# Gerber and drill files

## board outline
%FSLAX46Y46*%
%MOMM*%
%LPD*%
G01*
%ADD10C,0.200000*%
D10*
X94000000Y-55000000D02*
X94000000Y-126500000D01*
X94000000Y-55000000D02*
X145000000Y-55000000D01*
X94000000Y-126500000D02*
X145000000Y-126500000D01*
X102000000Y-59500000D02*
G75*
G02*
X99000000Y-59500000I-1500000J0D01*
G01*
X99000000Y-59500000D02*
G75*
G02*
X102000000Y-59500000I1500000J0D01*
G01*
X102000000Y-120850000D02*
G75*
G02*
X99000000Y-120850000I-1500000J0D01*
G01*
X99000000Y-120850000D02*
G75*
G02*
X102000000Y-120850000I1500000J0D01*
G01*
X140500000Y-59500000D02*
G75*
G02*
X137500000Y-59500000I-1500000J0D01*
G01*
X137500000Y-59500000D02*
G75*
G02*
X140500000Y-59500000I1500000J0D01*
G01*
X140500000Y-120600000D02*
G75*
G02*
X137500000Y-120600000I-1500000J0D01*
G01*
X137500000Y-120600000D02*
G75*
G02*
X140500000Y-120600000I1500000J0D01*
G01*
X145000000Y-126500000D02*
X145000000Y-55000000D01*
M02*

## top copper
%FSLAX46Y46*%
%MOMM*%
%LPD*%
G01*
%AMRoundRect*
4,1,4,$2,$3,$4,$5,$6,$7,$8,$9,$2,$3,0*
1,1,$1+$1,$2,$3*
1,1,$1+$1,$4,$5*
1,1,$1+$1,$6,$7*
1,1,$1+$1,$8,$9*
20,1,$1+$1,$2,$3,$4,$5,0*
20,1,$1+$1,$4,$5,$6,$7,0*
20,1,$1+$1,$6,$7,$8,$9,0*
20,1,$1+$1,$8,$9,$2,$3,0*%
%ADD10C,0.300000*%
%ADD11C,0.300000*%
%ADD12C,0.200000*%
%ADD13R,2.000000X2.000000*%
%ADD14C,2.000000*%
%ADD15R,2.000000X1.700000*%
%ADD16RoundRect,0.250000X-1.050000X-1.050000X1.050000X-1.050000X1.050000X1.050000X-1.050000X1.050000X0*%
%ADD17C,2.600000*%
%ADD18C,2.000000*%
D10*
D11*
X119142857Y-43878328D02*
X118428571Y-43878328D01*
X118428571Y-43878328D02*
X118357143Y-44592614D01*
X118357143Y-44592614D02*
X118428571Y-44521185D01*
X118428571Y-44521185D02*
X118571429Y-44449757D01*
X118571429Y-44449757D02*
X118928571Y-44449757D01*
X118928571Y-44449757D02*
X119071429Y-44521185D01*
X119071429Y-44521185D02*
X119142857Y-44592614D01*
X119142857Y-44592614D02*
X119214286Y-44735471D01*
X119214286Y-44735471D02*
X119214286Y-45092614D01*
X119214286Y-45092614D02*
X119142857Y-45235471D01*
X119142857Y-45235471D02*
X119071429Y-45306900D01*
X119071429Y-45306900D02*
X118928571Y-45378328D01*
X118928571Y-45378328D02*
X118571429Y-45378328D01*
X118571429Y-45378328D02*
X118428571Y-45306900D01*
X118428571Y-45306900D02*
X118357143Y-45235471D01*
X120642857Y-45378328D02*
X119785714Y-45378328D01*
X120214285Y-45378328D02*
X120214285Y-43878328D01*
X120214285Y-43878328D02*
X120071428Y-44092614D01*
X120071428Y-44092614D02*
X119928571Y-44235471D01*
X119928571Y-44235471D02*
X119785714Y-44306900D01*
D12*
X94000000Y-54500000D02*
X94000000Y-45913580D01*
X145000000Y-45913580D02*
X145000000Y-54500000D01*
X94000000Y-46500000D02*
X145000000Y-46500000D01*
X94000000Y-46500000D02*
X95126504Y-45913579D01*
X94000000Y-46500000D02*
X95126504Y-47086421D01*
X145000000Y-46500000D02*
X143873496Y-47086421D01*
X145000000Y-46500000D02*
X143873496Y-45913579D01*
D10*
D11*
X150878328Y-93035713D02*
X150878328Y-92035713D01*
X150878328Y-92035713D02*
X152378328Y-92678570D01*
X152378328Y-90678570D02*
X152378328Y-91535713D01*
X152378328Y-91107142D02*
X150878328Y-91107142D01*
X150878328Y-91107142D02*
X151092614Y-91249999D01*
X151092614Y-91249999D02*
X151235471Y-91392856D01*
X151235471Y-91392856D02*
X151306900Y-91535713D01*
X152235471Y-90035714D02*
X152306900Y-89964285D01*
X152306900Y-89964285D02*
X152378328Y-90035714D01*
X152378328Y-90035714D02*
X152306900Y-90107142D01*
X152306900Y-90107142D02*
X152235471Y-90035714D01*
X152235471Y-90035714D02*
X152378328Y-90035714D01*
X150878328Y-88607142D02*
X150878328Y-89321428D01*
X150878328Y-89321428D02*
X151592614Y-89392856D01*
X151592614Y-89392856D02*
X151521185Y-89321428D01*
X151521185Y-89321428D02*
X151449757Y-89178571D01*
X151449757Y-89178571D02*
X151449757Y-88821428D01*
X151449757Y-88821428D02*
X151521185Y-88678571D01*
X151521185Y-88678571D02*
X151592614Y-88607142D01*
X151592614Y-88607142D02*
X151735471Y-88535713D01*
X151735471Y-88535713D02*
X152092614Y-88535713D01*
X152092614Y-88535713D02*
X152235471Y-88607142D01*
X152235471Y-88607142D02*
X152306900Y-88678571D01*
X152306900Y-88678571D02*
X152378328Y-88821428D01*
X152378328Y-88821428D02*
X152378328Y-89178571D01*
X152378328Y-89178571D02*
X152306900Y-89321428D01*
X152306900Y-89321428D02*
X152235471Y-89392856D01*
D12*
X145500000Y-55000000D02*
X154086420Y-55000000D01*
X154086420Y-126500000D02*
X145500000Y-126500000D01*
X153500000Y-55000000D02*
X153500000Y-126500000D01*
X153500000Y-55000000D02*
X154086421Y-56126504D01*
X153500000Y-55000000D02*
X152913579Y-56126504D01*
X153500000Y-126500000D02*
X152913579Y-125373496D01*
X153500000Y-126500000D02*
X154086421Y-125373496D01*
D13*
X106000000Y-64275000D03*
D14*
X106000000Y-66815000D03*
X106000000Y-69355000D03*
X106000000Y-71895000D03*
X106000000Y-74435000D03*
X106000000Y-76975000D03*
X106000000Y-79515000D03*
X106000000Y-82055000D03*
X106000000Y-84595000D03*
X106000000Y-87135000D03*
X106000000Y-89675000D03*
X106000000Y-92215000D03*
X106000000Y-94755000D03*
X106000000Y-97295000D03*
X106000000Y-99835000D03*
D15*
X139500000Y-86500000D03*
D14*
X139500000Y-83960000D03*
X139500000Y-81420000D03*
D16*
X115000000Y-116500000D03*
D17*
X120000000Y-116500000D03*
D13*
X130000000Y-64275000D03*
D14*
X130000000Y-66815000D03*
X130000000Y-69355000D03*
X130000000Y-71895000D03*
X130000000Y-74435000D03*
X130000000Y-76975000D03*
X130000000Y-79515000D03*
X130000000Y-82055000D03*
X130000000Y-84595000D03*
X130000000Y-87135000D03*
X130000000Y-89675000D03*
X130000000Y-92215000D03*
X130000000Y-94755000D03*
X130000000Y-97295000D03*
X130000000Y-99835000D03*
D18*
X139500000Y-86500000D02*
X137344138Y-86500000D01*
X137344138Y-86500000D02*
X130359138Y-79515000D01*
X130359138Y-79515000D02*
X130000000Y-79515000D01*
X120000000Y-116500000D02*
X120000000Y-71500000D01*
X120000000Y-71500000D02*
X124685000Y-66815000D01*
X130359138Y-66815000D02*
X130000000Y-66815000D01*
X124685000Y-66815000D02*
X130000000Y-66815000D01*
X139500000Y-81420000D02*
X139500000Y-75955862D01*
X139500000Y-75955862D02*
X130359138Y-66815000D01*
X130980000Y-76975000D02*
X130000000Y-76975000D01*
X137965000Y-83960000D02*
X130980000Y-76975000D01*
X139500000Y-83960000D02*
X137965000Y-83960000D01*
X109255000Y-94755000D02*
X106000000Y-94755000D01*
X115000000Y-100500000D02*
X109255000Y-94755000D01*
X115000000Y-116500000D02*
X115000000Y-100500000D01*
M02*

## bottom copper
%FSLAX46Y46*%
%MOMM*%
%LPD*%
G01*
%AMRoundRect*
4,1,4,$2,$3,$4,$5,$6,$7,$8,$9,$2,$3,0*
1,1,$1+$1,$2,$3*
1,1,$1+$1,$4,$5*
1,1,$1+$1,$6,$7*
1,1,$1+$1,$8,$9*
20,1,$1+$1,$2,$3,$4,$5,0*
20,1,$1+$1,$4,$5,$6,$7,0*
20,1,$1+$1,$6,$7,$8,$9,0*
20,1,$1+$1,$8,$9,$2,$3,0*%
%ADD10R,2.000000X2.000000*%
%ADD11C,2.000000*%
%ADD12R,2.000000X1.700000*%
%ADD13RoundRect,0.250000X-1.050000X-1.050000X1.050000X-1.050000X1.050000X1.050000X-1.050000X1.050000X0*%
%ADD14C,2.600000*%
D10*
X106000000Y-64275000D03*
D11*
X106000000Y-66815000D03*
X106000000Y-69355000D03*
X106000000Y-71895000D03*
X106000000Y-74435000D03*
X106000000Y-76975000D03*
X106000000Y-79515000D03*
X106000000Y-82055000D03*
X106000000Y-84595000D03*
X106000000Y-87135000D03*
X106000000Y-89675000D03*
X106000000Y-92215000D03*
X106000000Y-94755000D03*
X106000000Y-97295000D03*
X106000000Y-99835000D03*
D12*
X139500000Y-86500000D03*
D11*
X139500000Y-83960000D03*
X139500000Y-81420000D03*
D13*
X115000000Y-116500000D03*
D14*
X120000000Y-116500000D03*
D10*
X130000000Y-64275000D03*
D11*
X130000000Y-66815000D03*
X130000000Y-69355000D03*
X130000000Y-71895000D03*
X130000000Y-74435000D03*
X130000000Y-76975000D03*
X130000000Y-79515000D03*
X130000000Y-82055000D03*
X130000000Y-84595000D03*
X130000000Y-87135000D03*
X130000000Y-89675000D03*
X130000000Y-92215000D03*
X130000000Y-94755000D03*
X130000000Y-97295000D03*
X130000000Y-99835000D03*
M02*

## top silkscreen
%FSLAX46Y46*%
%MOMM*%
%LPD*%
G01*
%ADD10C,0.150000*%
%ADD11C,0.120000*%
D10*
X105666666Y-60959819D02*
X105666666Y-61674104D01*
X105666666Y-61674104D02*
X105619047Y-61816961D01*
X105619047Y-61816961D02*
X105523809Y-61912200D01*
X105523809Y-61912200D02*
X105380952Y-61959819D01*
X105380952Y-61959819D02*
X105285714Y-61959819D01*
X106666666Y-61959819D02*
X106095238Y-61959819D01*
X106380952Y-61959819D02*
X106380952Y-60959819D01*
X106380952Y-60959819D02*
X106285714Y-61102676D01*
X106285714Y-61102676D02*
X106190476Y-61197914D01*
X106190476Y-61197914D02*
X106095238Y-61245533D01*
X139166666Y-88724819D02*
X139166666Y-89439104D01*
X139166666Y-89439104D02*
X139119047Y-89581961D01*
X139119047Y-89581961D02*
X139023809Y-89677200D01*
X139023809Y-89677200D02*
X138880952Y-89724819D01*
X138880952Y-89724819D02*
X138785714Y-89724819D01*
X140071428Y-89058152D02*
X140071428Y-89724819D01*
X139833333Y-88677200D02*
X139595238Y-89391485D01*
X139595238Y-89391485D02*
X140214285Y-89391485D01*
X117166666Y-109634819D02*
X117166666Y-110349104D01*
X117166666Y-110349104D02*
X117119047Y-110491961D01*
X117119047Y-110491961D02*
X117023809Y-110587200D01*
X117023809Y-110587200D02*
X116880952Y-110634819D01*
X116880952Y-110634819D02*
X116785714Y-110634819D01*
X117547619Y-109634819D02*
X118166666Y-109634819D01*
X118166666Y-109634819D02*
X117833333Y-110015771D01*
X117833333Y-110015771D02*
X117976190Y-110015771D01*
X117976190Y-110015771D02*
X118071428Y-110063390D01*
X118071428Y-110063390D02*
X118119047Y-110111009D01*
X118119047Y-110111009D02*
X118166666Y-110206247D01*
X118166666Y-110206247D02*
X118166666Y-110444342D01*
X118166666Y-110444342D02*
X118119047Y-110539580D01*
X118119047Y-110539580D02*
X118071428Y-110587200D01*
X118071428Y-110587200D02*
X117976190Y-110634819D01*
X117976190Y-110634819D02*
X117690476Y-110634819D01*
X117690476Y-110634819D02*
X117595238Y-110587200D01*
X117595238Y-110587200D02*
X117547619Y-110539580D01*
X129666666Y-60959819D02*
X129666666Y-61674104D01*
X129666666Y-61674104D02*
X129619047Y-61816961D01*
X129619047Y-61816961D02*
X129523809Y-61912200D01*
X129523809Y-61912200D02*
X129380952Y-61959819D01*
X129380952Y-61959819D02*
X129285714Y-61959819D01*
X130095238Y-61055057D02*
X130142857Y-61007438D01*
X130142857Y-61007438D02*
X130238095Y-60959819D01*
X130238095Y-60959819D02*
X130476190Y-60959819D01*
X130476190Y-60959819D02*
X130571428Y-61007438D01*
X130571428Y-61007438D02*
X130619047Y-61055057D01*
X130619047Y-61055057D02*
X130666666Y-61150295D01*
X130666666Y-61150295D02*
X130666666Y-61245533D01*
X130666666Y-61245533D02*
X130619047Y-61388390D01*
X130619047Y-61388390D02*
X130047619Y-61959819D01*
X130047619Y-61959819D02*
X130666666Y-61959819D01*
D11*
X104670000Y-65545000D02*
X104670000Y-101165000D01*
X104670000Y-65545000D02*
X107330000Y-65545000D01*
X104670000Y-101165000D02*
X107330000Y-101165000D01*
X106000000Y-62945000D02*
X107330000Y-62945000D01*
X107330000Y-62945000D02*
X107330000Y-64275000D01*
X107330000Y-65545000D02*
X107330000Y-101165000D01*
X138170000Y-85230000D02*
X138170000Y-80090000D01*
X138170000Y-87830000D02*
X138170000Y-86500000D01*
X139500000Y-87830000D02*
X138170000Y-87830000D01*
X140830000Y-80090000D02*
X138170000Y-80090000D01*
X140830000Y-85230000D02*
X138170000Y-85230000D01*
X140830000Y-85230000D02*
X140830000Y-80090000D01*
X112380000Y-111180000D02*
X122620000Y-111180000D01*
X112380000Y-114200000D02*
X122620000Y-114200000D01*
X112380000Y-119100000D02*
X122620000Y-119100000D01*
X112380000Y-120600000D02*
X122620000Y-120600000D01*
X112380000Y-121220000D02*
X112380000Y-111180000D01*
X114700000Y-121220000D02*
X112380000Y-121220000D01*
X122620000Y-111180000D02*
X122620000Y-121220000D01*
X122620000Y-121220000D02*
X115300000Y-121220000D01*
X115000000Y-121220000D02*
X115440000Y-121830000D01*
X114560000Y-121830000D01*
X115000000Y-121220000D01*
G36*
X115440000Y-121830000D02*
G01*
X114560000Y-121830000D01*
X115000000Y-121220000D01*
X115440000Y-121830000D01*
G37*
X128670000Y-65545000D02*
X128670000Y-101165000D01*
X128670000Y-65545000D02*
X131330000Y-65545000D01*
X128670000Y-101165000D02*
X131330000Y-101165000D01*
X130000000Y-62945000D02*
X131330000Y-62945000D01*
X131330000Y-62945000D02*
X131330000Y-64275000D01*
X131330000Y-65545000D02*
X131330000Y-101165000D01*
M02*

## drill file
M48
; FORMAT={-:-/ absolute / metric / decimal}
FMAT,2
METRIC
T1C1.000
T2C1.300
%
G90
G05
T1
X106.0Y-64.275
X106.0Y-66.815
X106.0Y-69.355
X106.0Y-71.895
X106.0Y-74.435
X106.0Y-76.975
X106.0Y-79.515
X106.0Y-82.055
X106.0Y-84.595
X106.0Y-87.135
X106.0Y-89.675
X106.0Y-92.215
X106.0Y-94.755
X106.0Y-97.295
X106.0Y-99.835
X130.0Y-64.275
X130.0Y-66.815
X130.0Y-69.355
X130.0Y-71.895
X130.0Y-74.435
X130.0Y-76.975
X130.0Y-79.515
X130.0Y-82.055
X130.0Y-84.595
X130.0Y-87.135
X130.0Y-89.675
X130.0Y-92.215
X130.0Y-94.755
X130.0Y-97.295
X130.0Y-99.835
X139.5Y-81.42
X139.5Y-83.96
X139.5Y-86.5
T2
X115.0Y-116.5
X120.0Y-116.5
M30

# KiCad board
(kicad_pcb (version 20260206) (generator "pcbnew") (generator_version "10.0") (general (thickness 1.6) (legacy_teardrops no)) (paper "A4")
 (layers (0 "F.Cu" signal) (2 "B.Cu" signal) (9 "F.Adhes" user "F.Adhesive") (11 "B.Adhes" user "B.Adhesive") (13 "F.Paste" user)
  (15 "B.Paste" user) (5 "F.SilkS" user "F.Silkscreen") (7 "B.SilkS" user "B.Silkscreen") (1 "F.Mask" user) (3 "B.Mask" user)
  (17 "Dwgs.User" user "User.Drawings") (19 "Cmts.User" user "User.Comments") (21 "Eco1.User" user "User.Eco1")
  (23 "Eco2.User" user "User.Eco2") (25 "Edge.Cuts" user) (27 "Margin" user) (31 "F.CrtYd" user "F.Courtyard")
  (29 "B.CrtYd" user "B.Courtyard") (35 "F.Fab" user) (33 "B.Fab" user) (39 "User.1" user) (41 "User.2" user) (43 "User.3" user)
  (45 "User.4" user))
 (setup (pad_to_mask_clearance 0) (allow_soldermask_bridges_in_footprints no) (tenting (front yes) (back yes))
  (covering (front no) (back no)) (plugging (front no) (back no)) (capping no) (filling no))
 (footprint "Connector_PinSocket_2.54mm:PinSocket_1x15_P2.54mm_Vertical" (layer "F.Cu") (at 106 64.275)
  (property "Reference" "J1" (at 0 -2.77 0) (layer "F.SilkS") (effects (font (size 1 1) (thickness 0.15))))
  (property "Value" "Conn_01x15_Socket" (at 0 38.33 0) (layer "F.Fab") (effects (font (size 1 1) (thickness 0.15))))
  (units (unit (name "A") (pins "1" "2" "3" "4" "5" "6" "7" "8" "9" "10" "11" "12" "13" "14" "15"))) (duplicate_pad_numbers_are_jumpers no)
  (fp_line (start -1.33 1.27) (end -1.33 36.89) (stroke (width 0.12) (type solid)) (layer "F.SilkS"))
  (fp_line (start -1.33 1.27) (end 1.33 1.27) (stroke (width 0.12) (type solid)) (layer "F.SilkS"))
  (fp_line (start -1.33 36.89) (end 1.33 36.89) (stroke (width 0.12) (type solid)) (layer "F.SilkS"))
  (fp_line (start 0 -1.33) (end 1.33 -1.33) (stroke (width 0.12) (type solid)) (layer "F.SilkS"))
  (fp_line (start 1.33 -1.33) (end 1.33 0) (stroke (width 0.12) (type solid)) (layer "F.SilkS"))
  (fp_line (start 1.33 1.27) (end 1.33 36.89) (stroke (width 0.12) (type solid)) (layer "F.SilkS"))
  (pad "1" thru_hole rect (at 0 0) (size 2 2) (drill 1) (layers "*.Cu" "*.Mask") (remove_unused_layers no)
   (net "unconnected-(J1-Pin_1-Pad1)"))
  (pad "2" thru_hole circle (at 0 2.54) (size 2 2) (drill 1) (layers "*.Cu" "*.Mask") (remove_unused_layers no)
   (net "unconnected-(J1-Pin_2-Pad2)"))
  (pad "3" thru_hole circle (at 0 5.08) (size 2 2) (drill 1) (layers "*.Cu" "*.Mask") (remove_unused_layers no)
   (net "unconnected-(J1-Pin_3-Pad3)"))
  (pad "4" thru_hole circle (at 0 7.62) (size 2 2) (drill 1) (layers "*.Cu" "*.Mask") (remove_unused_layers no)
   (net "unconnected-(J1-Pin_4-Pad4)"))
  (pad "5" thru_hole circle (at 0 10.16) (size 2 2) (drill 1) (layers "*.Cu" "*.Mask") (remove_unused_layers no)
   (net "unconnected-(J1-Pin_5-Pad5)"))
  (pad "6" thru_hole circle (at 0 12.7) (size 2 2) (drill 1) (layers "*.Cu" "*.Mask") (remove_unused_layers no)
   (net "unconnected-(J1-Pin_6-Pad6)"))
  (pad "7" thru_hole circle (at 0 15.24) (size 2 2) (drill 1) (layers "*.Cu" "*.Mask") (remove_unused_layers no)
   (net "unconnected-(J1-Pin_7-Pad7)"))
  (pad "8" thru_hole circle (at 0 17.78) (size 2 2) (drill 1) (layers "*.Cu" "*.Mask") (remove_unused_layers no)
   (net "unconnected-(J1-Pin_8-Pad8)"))
  (pad "9" thru_hole circle (at 0 20.32) (size 2 2) (drill 1) (layers "*.Cu" "*.Mask") (remove_unused_layers no)
   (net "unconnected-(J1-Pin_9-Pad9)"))
  (pad "10" thru_hole circle (at 0 22.86) (size 2 2) (drill 1) (layers "*.Cu" "*.Mask") (remove_unused_layers no)
   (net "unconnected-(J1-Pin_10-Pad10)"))
  (pad "11" thru_hole circle (at 0 25.4) (size 2 2) (drill 1) (layers "*.Cu" "*.Mask") (remove_unused_layers no)
   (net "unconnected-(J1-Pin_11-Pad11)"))
  (pad "12" thru_hole circle (at 0 27.94) (size 2 2) (drill 1) (layers "*.Cu" "*.Mask") (remove_unused_layers no)
   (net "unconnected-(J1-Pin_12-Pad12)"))
  (pad "13" thru_hole circle (at 0 30.48) (size 2 2) (drill 1) (layers "*.Cu" "*.Mask") (remove_unused_layers no) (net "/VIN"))
  (pad "14" thru_hole circle (at 0 33.02) (size 2 2) (drill 1) (layers "*.Cu" "*.Mask") (remove_unused_layers no)
   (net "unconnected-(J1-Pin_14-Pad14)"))
  (pad "15" thru_hole circle (at 0 35.56) (size 2 2) (drill 1) (layers "*.Cu" "*.Mask") (remove_unused_layers no)
   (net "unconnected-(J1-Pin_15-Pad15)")))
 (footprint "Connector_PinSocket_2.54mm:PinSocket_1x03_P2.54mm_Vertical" (layer "F.Cu") (at 139.5 86.5 180)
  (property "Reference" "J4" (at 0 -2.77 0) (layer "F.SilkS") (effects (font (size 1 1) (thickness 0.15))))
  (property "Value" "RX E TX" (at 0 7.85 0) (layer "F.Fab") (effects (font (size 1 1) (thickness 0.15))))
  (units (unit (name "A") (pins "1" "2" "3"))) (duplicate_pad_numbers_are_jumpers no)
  (fp_line (start 1.33 1.27) (end 1.33 6.41) (stroke (width 0.12) (type solid)) (layer "F.SilkS"))
  (fp_line (start 1.33 -1.33) (end 1.33 0) (stroke (width 0.12) (type solid)) (layer "F.SilkS"))
  (fp_line (start 0 -1.33) (end 1.33 -1.33) (stroke (width 0.12) (type solid)) (layer "F.SilkS"))
  (fp_line (start -1.33 6.41) (end 1.33 6.41) (stroke (width 0.12) (type solid)) (layer "F.SilkS"))
  (fp_line (start -1.33 1.27) (end 1.33 1.27) (stroke (width 0.12) (type solid)) (layer "F.SilkS"))
  (fp_line (start -1.33 1.27) (end -1.33 6.41) (stroke (width 0.12) (type solid)) (layer "F.SilkS"))
  (pad "1" thru_hole rect (at 0 0 180) (size 2 1.7) (drill 1) (layers "*.Cu" "*.Mask") (remove_unused_layers no) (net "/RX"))
  (pad "2" thru_hole circle (at 0 2.54 180) (size 2 2) (drill 1) (layers "*.Cu" "*.Mask") (remove_unused_layers no) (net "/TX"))
  (pad "3" thru_hole circle (at 0 5.08 180) (size 2 2) (drill 1) (layers "*.Cu" "*.Mask") (remove_unused_layers no) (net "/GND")))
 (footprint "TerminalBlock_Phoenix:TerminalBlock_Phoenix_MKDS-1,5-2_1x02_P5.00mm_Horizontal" (layer "F.Cu") (at 115 116.5)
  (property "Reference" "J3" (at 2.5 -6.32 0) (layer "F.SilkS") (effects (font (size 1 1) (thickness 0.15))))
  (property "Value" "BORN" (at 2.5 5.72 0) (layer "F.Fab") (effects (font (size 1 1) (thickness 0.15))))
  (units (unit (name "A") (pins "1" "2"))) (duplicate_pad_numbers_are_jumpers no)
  (fp_line (start -2.62 -5.32) (end 7.62 -5.32) (stroke (width 0.12) (type solid)) (layer "F.SilkS"))
  (fp_line (start -2.62 -2.3) (end 7.62 -2.3) (stroke (width 0.12) (type solid)) (layer "F.SilkS"))
  (fp_line (start -2.62 2.6) (end 7.62 2.6) (stroke (width 0.12) (type solid)) (layer "F.SilkS"))
  (fp_line (start -2.62 4.1) (end 7.62 4.1) (stroke (width 0.12) (type solid)) (layer "F.SilkS"))
  (fp_line (start -2.62 4.72) (end -2.62 -5.32) (stroke (width 0.12) (type solid)) (layer "F.SilkS"))
  (fp_line (start -0.3 4.72) (end -2.62 4.72) (stroke (width 0.12) (type solid)) (layer "F.SilkS"))
  (fp_line (start 7.62 -5.32) (end 7.62 4.72) (stroke (width 0.12) (type solid)) (layer "F.SilkS"))
  (fp_line (start 7.62 4.72) (end 0.3 4.72) (stroke (width 0.12) (type solid)) (layer "F.SilkS"))
  (fp_poly (pts (xy 0 4.72) (xy 0.44 5.33) (xy -0.44 5.33)) (stroke (width 0.12) (type solid)) (fill yes) (layer "F.SilkS"))
  (pad "1" thru_hole roundrect (at 0 0) (size 2.6 2.6) (drill 1.3) (layers "*.Cu" "*.Mask") (remove_unused_layers no)
   (roundrect_rratio 0.096154) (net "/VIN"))
  (pad "2" thru_hole circle (at 5 0) (size 2.6 2.6) (drill 1.3) (layers "*.Cu" "*.Mask") (remove_unused_layers no) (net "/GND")))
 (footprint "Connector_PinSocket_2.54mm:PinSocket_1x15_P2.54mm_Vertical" (layer "F.Cu") (at 130 64.275)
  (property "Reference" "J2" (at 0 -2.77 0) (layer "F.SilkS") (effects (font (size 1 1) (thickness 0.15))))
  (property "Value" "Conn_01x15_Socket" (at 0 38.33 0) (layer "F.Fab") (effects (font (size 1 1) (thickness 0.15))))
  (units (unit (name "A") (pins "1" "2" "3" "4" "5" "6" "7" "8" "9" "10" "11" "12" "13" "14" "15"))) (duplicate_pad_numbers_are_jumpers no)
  (fp_line (start -1.33 1.27) (end -1.33 36.89) (stroke (width 0.12) (type solid)) (layer "F.SilkS"))
  (fp_line (start -1.33 1.27) (end 1.33 1.27) (stroke (width 0.12) (type solid)) (layer "F.SilkS"))
  (fp_line (start -1.33 36.89) (end 1.33 36.89) (stroke (width 0.12) (type solid)) (layer "F.SilkS"))
  (fp_line (start 0 -1.33) (end 1.33 -1.33) (stroke (width 0.12) (type solid)) (layer "F.SilkS"))
  (fp_line (start 1.33 -1.33) (end 1.33 0) (stroke (width 0.12) (type solid)) (layer "F.SilkS"))
  (fp_line (start 1.33 1.27) (end 1.33 36.89) (stroke (width 0.12) (type solid)) (layer "F.SilkS"))
  (pad "1" thru_hole rect (at 0 0) (size 2 2) (drill 1) (layers "*.Cu" "*.Mask") (remove_unused_layers no)
   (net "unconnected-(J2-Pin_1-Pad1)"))
  (pad "2" thru_hole circle (at 0 2.54) (size 2 2) (drill 1) (layers "*.Cu" "*.Mask") (remove_unused_layers no) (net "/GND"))
  (pad "3" thru_hole circle (at 0 5.08) (size 2 2) (drill 1) (layers "*.Cu" "*.Mask") (remove_unused_layers no)
   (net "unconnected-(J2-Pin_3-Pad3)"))
  (pad "4" thru_hole circle (at 0 7.62) (size 2 2) (drill 1) (layers "*.Cu" "*.Mask") (remove_unused_layers no)
   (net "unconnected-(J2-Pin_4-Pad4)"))
  (pad "5" thru_hole circle (at 0 10.16) (size 2 2) (drill 1) (layers "*.Cu" "*.Mask") (remove_unused_layers no)
   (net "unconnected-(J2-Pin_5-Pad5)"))
  (pad "6" thru_hole circle (at 0 12.7) (size 2 2) (drill 1) (layers "*.Cu" "*.Mask") (remove_unused_layers no) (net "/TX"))
  (pad "7" thru_hole circle (at 0 15.24) (size 2 2) (drill 1) (layers "*.Cu" "*.Mask") (remove_unused_layers no) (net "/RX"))
  (pad "8" thru_hole circle (at 0 17.78) (size 2 2) (drill 1) (layers "*.Cu" "*.Mask") (remove_unused_layers no)
   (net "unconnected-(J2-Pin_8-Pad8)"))
  (pad "9" thru_hole circle (at 0 20.32) (size 2 2) (drill 1) (layers "*.Cu" "*.Mask") (remove_unused_layers no)
   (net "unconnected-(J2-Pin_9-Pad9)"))
  (pad "10" thru_hole circle (at 0 22.86) (size 2 2) (drill 1) (layers "*.Cu" "*.Mask") (remove_unused_layers no)
   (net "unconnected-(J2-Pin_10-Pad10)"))
  (pad "11" thru_hole circle (at 0 25.4) (size 2 2) (drill 1) (layers "*.Cu" "*.Mask") (remove_unused_layers no)
   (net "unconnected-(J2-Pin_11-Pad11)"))
  (pad "12" thru_hole circle (at 0 27.94) (size 2 2) (drill 1) (layers "*.Cu" "*.Mask") (remove_unused_layers no)
   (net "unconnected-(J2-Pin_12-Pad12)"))
  (pad "13" thru_hole circle (at 0 30.48) (size 2 2) (drill 1) (layers "*.Cu" "*.Mask") (remove_unused_layers no)
   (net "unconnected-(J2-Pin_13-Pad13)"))
  (pad "14" thru_hole circle (at 0 33.02) (size 2 2) (drill 1) (layers "*.Cu" "*.Mask") (remove_unused_layers no)
   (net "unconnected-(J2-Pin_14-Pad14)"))
  (pad "15" thru_hole circle (at 0 35.56) (size 2 2) (drill 1) (layers "*.Cu" "*.Mask") (remove_unused_layers no)
   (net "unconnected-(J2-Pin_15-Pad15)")))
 (gr_line (start 94 55) (end 94 126.5) (stroke (width 0.2) (type solid)) (layer "Edge.Cuts"))
 (gr_line (start 94 55) (end 145 55) (stroke (width 0.2) (type solid)) (layer "Edge.Cuts"))
 (gr_line (start 94 126.5) (end 145 126.5) (stroke (width 0.2) (type solid)) (layer "Edge.Cuts"))
 (gr_circle (center 100.5 59.5) (end 100.5 58) (stroke (width 0.2) (type solid)) (fill no) (layer "Edge.Cuts"))
 (gr_circle (center 100.5 120.85) (end 99 120.85) (stroke (width 0.2) (type solid)) (fill no) (layer "Edge.Cuts"))
 (gr_circle (center 139 59.5) (end 137.5 59.5) (stroke (width 0.2) (type solid)) (fill no) (layer "Edge.Cuts"))
 (gr_circle (center 139 120.6) (end 137.5 120.6) (stroke (width 0.2) (type solid)) (fill no) (layer "Edge.Cuts"))
 (gr_line (start 145 126.5) (end 145 55) (stroke (width 0.2) (type solid)) (layer "Edge.Cuts"))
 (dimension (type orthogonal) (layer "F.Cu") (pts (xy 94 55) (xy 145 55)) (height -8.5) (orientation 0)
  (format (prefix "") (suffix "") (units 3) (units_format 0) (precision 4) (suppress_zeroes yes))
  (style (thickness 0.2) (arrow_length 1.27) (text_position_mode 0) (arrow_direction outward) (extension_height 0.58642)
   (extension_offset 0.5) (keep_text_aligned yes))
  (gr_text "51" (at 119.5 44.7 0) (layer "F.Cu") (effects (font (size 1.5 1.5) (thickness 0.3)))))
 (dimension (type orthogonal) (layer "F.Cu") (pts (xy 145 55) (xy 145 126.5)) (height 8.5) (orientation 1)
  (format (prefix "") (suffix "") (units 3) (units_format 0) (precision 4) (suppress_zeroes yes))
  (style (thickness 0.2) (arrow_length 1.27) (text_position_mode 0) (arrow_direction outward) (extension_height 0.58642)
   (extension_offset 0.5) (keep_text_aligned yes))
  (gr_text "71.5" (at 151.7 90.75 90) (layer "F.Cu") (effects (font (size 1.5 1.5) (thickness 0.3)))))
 (segment (start 139.5 86.5) (end 137.344138 86.5) (width 2) (layer "F.Cu") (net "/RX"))
 (segment (start 137.344138 86.5) (end 130.359138 79.515) (width 2) (layer "F.Cu") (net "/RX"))
 (segment (start 130.359138 79.515) (end 130 79.515) (width 2) (layer "F.Cu") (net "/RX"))
 (segment (start 120 116.5) (end 120 71.5) (width 2) (layer "F.Cu") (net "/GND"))
 (segment (start 120 71.5) (end 124.685 66.815) (width 2) (layer "F.Cu") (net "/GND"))
 (segment (start 130.359138 66.815) (end 130 66.815) (width 2) (layer "F.Cu") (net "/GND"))
 (segment (start 124.685 66.815) (end 130 66.815) (width 2) (layer "F.Cu") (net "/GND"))
 (segment (start 139.5 81.42) (end 139.5 75.955862) (width 2) (layer "F.Cu") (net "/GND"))
 (segment (start 139.5 75.955862) (end 130.359138 66.815) (width 2) (layer "F.Cu") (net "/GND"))
 (segment (start 130.98 76.975) (end 130 76.975) (width 2) (layer "F.Cu") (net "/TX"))
 (segment (start 137.965 83.96) (end 130.98 76.975) (width 2) (layer "F.Cu") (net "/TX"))
 (segment (start 139.5 83.96) (end 137.965 83.96) (width 2) (layer "F.Cu") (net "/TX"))
 (segment (start 109.255 94.755) (end 106 94.755) (width 2) (layer "F.Cu") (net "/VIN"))
 (segment (start 115 100.5) (end 109.255 94.755) (width 2) (layer "F.Cu") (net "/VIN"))
 (segment (start 115 116.5) (end 115 100.5) (width 2) (layer "F.Cu") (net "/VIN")))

